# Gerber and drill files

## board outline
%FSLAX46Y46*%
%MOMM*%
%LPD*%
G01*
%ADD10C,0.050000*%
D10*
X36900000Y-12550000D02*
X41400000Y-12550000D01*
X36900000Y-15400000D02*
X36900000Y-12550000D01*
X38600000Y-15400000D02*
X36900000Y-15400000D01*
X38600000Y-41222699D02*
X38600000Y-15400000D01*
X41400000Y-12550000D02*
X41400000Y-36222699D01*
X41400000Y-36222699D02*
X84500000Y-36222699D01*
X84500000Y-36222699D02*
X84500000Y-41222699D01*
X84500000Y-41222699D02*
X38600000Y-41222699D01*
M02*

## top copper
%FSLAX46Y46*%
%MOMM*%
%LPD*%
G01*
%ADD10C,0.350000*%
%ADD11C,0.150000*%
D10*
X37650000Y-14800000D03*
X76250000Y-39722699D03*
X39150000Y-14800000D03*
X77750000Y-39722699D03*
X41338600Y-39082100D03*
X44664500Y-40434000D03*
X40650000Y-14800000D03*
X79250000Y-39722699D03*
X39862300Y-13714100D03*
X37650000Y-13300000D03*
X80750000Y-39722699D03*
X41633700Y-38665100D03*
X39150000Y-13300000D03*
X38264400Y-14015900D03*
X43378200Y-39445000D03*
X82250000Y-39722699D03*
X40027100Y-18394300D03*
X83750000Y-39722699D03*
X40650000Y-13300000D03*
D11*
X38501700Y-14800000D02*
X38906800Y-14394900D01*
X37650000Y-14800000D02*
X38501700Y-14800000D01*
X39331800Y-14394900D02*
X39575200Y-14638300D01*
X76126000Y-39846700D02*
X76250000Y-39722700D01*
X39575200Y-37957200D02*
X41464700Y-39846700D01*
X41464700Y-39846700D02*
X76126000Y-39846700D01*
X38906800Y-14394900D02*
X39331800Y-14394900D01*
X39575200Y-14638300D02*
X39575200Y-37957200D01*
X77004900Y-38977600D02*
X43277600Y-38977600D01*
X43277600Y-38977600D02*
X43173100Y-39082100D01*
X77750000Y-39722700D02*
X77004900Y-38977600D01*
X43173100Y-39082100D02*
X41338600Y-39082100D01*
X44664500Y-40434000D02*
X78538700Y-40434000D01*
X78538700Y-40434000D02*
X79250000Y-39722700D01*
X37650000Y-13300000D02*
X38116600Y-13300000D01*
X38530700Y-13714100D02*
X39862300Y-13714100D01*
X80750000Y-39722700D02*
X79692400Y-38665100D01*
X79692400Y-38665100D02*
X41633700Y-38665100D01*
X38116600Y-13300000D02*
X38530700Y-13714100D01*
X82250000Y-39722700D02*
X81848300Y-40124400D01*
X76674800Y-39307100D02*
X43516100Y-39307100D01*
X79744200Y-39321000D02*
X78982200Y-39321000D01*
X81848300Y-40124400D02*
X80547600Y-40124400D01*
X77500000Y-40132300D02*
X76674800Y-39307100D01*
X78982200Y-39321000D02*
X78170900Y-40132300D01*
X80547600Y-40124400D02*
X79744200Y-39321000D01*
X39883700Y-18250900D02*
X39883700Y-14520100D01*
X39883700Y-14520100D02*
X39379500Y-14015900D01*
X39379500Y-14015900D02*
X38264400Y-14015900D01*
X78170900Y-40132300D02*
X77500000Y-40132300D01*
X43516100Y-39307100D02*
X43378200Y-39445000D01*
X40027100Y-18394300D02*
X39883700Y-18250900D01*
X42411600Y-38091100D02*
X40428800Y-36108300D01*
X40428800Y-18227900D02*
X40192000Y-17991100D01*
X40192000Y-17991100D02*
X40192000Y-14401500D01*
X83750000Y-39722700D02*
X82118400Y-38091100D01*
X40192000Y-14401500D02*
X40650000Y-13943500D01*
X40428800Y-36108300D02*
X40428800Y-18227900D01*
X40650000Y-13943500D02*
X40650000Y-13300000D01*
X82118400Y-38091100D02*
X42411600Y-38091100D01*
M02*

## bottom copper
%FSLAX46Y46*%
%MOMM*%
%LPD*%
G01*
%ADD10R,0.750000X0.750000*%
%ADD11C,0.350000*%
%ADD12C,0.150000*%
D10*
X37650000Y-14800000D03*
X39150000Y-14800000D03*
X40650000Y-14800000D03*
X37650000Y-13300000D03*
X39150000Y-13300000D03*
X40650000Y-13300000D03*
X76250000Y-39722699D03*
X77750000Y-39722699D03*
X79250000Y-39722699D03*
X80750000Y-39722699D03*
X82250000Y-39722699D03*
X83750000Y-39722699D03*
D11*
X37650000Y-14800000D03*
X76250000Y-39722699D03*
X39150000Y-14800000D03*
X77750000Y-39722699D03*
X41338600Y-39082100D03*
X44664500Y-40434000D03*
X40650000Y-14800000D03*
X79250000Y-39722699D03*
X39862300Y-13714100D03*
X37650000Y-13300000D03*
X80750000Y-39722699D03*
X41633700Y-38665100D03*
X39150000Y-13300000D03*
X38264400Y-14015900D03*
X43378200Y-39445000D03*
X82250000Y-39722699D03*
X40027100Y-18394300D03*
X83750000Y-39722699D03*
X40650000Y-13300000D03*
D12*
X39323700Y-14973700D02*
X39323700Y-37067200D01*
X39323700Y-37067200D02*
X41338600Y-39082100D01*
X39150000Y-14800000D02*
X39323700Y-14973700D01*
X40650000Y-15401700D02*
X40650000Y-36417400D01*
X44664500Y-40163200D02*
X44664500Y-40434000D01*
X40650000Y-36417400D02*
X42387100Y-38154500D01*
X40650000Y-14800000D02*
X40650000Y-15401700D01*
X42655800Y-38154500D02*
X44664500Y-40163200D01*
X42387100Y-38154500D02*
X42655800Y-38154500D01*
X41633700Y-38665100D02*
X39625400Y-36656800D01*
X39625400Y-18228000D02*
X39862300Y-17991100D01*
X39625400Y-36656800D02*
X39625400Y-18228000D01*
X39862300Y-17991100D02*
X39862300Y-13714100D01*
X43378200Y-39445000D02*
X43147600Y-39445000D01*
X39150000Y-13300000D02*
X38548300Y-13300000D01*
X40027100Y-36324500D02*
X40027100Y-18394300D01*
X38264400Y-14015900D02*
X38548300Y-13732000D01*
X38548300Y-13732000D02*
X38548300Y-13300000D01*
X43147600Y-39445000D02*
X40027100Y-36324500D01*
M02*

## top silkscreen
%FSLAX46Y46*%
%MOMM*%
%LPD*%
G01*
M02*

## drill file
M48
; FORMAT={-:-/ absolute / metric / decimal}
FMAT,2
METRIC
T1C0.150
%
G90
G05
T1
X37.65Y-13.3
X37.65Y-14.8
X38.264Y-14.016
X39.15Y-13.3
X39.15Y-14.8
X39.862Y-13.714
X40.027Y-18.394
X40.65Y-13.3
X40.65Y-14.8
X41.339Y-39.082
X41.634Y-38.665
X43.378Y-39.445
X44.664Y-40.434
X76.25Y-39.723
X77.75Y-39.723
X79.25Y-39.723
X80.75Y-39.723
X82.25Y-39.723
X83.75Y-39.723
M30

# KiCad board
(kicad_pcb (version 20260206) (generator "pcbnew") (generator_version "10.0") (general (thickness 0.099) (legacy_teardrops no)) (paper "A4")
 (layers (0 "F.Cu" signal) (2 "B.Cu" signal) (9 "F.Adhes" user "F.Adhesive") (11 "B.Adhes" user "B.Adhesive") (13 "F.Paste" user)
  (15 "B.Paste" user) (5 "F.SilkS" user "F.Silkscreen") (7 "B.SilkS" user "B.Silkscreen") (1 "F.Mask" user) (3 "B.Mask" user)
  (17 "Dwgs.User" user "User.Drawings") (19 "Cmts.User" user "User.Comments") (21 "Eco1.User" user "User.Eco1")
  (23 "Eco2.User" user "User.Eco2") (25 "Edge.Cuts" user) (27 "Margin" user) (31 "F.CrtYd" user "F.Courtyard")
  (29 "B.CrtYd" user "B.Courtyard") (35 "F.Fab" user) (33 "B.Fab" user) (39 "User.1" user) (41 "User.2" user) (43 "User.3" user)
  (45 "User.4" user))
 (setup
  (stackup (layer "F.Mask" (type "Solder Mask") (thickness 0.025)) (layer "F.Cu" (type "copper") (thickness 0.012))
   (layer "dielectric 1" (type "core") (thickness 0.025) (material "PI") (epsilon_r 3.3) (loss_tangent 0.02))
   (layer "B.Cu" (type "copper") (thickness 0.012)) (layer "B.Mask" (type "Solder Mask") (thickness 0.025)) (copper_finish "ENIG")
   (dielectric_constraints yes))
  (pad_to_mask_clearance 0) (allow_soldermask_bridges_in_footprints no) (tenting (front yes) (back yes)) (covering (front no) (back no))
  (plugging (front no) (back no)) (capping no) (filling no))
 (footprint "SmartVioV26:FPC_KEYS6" (layer "F.Cu") (at 0 0)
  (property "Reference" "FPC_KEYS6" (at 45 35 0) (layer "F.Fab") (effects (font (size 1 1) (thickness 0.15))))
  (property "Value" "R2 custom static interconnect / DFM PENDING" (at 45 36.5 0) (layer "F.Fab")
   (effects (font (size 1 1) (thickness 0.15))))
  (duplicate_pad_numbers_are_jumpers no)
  (pad "S1" smd rect (at 37.65 14.8) (size 0.75 0.75) (layers "B.Cu" "B.Mask") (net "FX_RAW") (solder_mask_margin 0.1))
  (pad "S2" smd rect (at 39.15 14.8) (size 0.75 0.75) (layers "B.Cu" "B.Mask") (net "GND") (solder_mask_margin 0.1))
  (pad "S3" smd rect (at 40.65 14.8) (size 0.75 0.75) (layers "B.Cu" "B.Mask") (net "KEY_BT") (solder_mask_margin 0.1))
  (pad "S4" smd rect (at 37.65 13.3) (size 0.75 0.75) (layers "B.Cu" "B.Mask") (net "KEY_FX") (solder_mask_margin 0.1))
  (pad "S5" smd rect (at 39.15 13.3) (size 0.75 0.75) (layers "B.Cu" "B.Mask") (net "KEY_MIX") (solder_mask_margin 0.1))
  (pad "S6" smd rect (at 40.65 13.3) (size 0.75 0.75) (layers "B.Cu" "B.Mask") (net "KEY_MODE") (solder_mask_margin 0.1))
  (pad "T1" smd rect (at 76.25 39.722699) (size 0.75 0.75) (layers "B.Cu" "B.Mask") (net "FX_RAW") (solder_mask_margin 0.1))
  (pad "T2" smd rect (at 77.75 39.722699) (size 0.75 0.75) (layers "B.Cu" "B.Mask") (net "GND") (solder_mask_margin 0.1))
  (pad "T3" smd rect (at 79.25 39.722699) (size 0.75 0.75) (layers "B.Cu" "B.Mask") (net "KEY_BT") (solder_mask_margin 0.1))
  (pad "T4" smd rect (at 80.75 39.722699) (size 0.75 0.75) (layers "B.Cu" "B.Mask") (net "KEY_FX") (solder_mask_margin 0.1))
  (pad "T5" smd rect (at 82.25 39.722699) (size 0.75 0.75) (layers "B.Cu" "B.Mask") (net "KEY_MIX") (solder_mask_margin 0.1))
  (pad "T6" smd rect (at 83.75 39.722699) (size 0.75 0.75) (layers "B.Cu" "B.Mask") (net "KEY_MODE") (solder_mask_margin 0.1)))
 (gr_line (start 36.9 12.55) (end 41.4 12.55) (stroke (width 0.05) (type default)) (layer "Edge.Cuts"))
 (gr_line (start 36.9 15.4) (end 36.9 12.55) (stroke (width 0.05) (type default)) (layer "Edge.Cuts"))
 (gr_line (start 38.6 15.4) (end 36.9 15.4) (stroke (width 0.05) (type default)) (layer "Edge.Cuts"))
 (gr_line (start 38.6 41.222699) (end 38.6 15.4) (stroke (width 0.05) (type default)) (layer "Edge.Cuts"))
 (gr_line (start 41.4 12.55) (end 41.4 36.222699) (stroke (width 0.05) (type default)) (layer "Edge.Cuts"))
 (gr_line (start 41.4 36.222699) (end 84.5 36.222699) (stroke (width 0.05) (type default)) (layer "Edge.Cuts"))
 (gr_line (start 84.5 36.222699) (end 84.5 41.222699) (stroke (width 0.05) (type default)) (layer "Edge.Cuts"))
 (gr_line (start 84.5 41.222699) (end 38.6 41.222699) (stroke (width 0.05) (type default)) (layer "Edge.Cuts"))
 (segment (start 38.5017 14.8) (end 38.9068 14.3949) (width 0.15) (layer "F.Cu") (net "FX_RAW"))
 (segment (start 37.65 14.8) (end 38.5017 14.8) (width 0.15) (layer "F.Cu") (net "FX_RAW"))
 (segment (start 39.3318 14.3949) (end 39.5752 14.6383) (width 0.15) (layer "F.Cu") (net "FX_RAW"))
 (segment (start 76.126 39.8467) (end 76.25 39.7227) (width 0.15) (layer "F.Cu") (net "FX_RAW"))
 (segment (start 39.5752 37.9572) (end 41.4647 39.8467) (width 0.15) (layer "F.Cu") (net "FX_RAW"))
 (segment (start 41.4647 39.8467) (end 76.126 39.8467) (width 0.15) (layer "F.Cu") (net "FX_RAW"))
 (segment (start 38.9068 14.3949) (end 39.3318 14.3949) (width 0.15) (layer "F.Cu") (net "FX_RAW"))
 (segment (start 39.5752 14.6383) (end 39.5752 37.9572) (width 0.15) (layer "F.Cu") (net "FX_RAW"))
 (via (at 37.65 14.8) (size 0.35) (drill 0.15) (layers "F.Cu" "B.Cu") (locked yes) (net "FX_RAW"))
 (via (at 76.25 39.722699) (size 0.35) (drill 0.15) (layers "F.Cu" "B.Cu") (locked yes) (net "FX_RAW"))
 (segment (start 77.0049 38.9776) (end 43.2776 38.9776) (width 0.15) (layer "F.Cu") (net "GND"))
 (segment (start 43.2776 38.9776) (end 43.1731 39.0821) (width 0.15) (layer "F.Cu") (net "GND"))
 (segment (start 77.75 39.7227) (end 77.0049 38.9776) (width 0.15) (layer "F.Cu") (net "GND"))
 (segment (start 43.1731 39.0821) (end 41.3386 39.0821) (width 0.15) (layer "F.Cu") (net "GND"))
 (via (at 39.15 14.8) (size 0.35) (drill 0.15) (layers "F.Cu" "B.Cu") (locked yes) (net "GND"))
 (via (at 77.75 39.722699) (size 0.35) (drill 0.15) (layers "F.Cu" "B.Cu") (locked yes) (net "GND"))
 (via (at 41.3386 39.0821) (size 0.35) (drill 0.15) (layers "F.Cu" "B.Cu") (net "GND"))
 (segment (start 39.3237 14.9737) (end 39.3237 37.0672) (width 0.15) (layer "B.Cu") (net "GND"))
 (segment (start 39.3237 37.0672) (end 41.3386 39.0821) (width 0.15) (layer "B.Cu") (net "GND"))
 (segment (start 39.15 14.8) (end 39.3237 14.9737) (width 0.15) (layer "B.Cu") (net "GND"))
 (segment (start 44.6645 40.434) (end 78.5387 40.434) (width 0.15) (layer "F.Cu") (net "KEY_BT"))
 (segment (start 78.5387 40.434) (end 79.25 39.7227) (width 0.15) (layer "F.Cu") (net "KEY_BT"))
 (via (at 44.6645 40.434) (size 0.35) (drill 0.15) (layers "F.Cu" "B.Cu") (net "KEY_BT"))
 (via (at 40.65 14.8) (size 0.35) (drill 0.15) (layers "F.Cu" "B.Cu") (locked yes) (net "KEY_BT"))
 (via (at 79.25 39.722699) (size 0.35) (drill 0.15) (layers "F.Cu" "B.Cu") (locked yes) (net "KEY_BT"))
 (segment (start 40.65 15.4017) (end 40.65 36.4174) (width 0.15) (layer "B.Cu") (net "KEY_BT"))
 (segment (start 44.6645 40.1632) (end 44.6645 40.434) (width 0.15) (layer "B.Cu") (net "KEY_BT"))
 (segment (start 40.65 36.4174) (end 42.3871 38.1545) (width 0.15) (layer "B.Cu") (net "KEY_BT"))
 (segment (start 40.65 14.8) (end 40.65 15.4017) (width 0.15) (layer "B.Cu") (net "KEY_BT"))
 (segment (start 42.6558 38.1545) (end 44.6645 40.1632) (width 0.15) (layer "B.Cu") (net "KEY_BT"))
 (segment (start 42.3871 38.1545) (end 42.6558 38.1545) (width 0.15) (layer "B.Cu") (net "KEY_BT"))
 (segment (start 37.65 13.3) (end 38.1166 13.3) (width 0.15) (layer "F.Cu") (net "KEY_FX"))
 (segment (start 38.5307 13.7141) (end 39.8623 13.7141) (width 0.15) (layer "F.Cu") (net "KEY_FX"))
 (segment (start 80.75 39.7227) (end 79.6924 38.6651) (width 0.15) (layer "F.Cu") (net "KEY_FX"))
 (segment (start 79.6924 38.6651) (end 41.6337 38.6651) (width 0.15) (layer "F.Cu") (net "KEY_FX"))
 (segment (start 38.1166 13.3) (end 38.5307 13.7141) (width 0.15) (layer "F.Cu") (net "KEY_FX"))
 (via (at 39.8623 13.7141) (size 0.35) (drill 0.15) (layers "F.Cu" "B.Cu") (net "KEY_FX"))
 (via (at 37.65 13.3) (size 0.35) (drill 0.15) (layers "F.Cu" "B.Cu") (locked yes) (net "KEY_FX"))
 (via (at 80.75 39.722699) (size 0.35) (drill 0.15) (layers "F.Cu" "B.Cu") (locked yes) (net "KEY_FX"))
 (via (at 41.6337 38.6651) (size 0.35) (drill 0.15) (layers "F.Cu" "B.Cu") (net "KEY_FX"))
 (segment (start 41.6337 38.6651) (end 39.6254 36.6568) (width 0.15) (layer "B.Cu") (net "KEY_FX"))
 (segment (start 39.6254 18.228) (end 39.8623 17.9911) (width 0.15) (layer "B.Cu") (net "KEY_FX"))
 (segment (start 39.6254 36.6568) (end 39.6254 18.228) (width 0.15) (layer "B.Cu") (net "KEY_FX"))
 (segment (start 39.8623 17.9911) (end 39.8623 13.7141) (width 0.15) (layer "B.Cu") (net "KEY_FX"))
 (segment (start 82.25 39.7227) (end 81.8483 40.1244) (width 0.15) (layer "F.Cu") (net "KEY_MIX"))
 (segment (start 76.6748 39.3071) (end 43.5161 39.3071) (width 0.15) (layer "F.Cu") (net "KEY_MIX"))
 (segment (start 79.7442 39.321) (end 78.9822 39.321) (width 0.15) (layer "F.Cu") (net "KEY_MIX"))
 (segment (start 81.8483 40.1244) (end 80.5476 40.1244) (width 0.15) (layer "F.Cu") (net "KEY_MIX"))
 (segment (start 77.5 40.1323) (end 76.6748 39.3071) (width 0.15) (layer "F.Cu") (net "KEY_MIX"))
 (segment (start 78.9822 39.321) (end 78.1709 40.1323) (width 0.15) (layer "F.Cu") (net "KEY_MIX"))
 (segment (start 80.5476 40.1244) (end 79.7442 39.321) (width 0.15) (layer "F.Cu") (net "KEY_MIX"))
 (segment (start 39.8837 18.2509) (end 39.8837 14.5201) (width 0.15) (layer "F.Cu") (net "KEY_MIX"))
 (segment (start 39.8837 14.5201) (end 39.3795 14.0159) (width 0.15) (layer "F.Cu") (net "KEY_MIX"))
 (segment (start 39.3795 14.0159) (end 38.2644 14.0159) (width 0.15) (layer "F.Cu") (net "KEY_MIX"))
 (segment (start 78.1709 40.1323) (end 77.5 40.1323) (width 0.15) (layer "F.Cu") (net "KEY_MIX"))
 (segment (start 43.5161 39.3071) (end 43.3782 39.445) (width 0.15) (layer "F.Cu") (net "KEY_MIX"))
 (segment (start 40.0271 18.3943) (end 39.8837 18.2509) (width 0.15) (layer "F.Cu") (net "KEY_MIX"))
 (via (at 39.15 13.3) (size 0.35) (drill 0.15) (layers "F.Cu" "B.Cu") (locked yes) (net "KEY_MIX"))
 (via (at 38.2644 14.0159) (size 0.35) (drill 0.15) (layers "F.Cu" "B.Cu") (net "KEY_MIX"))
 (via (at 43.3782 39.445) (size 0.35) (drill 0.15) (layers "F.Cu" "B.Cu") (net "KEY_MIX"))
 (via (at 82.25 39.722699) (size 0.35) (drill 0.15) (layers "F.Cu" "B.Cu") (locked yes) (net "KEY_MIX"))
 (via (at 40.0271 18.3943) (size 0.35) (drill 0.15) (layers "F.Cu" "B.Cu") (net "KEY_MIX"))
 (segment (start 43.3782 39.445) (end 43.1476 39.445) (width 0.15) (layer "B.Cu") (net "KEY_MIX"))
 (segment (start 39.15 13.3) (end 38.5483 13.3) (width 0.15) (layer "B.Cu") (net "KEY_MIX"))
 (segment (start 40.0271 36.3245) (end 40.0271 18.3943) (width 0.15) (layer "B.Cu") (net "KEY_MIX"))
 (segment (start 38.2644 14.0159) (end 38.5483 13.732) (width 0.15) (layer "B.Cu") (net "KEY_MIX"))
 (segment (start 38.5483 13.732) (end 38.5483 13.3) (width 0.15) (layer "B.Cu") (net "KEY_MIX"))
 (segment (start 43.1476 39.445) (end 40.0271 36.3245) (width 0.15) (layer "B.Cu") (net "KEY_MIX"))
 (segment (start 42.4116 38.0911) (end 40.4288 36.1083) (width 0.15) (layer "F.Cu") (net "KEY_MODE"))
 (segment (start 40.4288 18.2279) (end 40.192 17.9911) (width 0.15) (layer "F.Cu") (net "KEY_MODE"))
 (segment (start 40.192 17.9911) (end 40.192 14.4015) (width 0.15) (layer "F.Cu") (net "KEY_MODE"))
 (segment (start 83.75 39.7227) (end 82.1184 38.0911) (width 0.15) (layer "F.Cu") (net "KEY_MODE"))
 (segment (start 40.192 14.4015) (end 40.65 13.9435) (width 0.15) (layer "F.Cu") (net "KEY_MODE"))
 (segment (start 40.4288 36.1083) (end 40.4288 18.2279) (width 0.15) (layer "F.Cu") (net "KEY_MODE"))
 (segment (start 40.65 13.9435) (end 40.65 13.3) (width 0.15) (layer "F.Cu") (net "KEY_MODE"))
 (segment (start 82.1184 38.0911) (end 42.4116 38.0911) (width 0.15) (layer "F.Cu") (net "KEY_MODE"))
 (via (at 83.75 39.722699) (size 0.35) (drill 0.15) (layers "F.Cu" "B.Cu") (locked yes) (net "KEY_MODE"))
 (via (at 40.65 13.3) (size 0.35) (drill 0.15) (layers "F.Cu" "B.Cu") (locked yes) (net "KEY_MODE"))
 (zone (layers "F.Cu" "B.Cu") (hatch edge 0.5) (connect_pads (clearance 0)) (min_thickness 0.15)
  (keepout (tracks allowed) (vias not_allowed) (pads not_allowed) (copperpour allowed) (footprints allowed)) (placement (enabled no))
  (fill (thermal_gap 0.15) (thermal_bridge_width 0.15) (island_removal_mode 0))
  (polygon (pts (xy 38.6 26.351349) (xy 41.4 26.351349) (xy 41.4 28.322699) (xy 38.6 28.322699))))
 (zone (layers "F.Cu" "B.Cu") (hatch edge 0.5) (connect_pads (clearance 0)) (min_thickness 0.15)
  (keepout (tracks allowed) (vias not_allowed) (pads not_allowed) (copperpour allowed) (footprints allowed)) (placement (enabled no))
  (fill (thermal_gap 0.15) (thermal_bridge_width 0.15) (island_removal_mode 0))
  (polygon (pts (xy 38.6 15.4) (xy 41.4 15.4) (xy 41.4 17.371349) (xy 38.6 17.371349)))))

